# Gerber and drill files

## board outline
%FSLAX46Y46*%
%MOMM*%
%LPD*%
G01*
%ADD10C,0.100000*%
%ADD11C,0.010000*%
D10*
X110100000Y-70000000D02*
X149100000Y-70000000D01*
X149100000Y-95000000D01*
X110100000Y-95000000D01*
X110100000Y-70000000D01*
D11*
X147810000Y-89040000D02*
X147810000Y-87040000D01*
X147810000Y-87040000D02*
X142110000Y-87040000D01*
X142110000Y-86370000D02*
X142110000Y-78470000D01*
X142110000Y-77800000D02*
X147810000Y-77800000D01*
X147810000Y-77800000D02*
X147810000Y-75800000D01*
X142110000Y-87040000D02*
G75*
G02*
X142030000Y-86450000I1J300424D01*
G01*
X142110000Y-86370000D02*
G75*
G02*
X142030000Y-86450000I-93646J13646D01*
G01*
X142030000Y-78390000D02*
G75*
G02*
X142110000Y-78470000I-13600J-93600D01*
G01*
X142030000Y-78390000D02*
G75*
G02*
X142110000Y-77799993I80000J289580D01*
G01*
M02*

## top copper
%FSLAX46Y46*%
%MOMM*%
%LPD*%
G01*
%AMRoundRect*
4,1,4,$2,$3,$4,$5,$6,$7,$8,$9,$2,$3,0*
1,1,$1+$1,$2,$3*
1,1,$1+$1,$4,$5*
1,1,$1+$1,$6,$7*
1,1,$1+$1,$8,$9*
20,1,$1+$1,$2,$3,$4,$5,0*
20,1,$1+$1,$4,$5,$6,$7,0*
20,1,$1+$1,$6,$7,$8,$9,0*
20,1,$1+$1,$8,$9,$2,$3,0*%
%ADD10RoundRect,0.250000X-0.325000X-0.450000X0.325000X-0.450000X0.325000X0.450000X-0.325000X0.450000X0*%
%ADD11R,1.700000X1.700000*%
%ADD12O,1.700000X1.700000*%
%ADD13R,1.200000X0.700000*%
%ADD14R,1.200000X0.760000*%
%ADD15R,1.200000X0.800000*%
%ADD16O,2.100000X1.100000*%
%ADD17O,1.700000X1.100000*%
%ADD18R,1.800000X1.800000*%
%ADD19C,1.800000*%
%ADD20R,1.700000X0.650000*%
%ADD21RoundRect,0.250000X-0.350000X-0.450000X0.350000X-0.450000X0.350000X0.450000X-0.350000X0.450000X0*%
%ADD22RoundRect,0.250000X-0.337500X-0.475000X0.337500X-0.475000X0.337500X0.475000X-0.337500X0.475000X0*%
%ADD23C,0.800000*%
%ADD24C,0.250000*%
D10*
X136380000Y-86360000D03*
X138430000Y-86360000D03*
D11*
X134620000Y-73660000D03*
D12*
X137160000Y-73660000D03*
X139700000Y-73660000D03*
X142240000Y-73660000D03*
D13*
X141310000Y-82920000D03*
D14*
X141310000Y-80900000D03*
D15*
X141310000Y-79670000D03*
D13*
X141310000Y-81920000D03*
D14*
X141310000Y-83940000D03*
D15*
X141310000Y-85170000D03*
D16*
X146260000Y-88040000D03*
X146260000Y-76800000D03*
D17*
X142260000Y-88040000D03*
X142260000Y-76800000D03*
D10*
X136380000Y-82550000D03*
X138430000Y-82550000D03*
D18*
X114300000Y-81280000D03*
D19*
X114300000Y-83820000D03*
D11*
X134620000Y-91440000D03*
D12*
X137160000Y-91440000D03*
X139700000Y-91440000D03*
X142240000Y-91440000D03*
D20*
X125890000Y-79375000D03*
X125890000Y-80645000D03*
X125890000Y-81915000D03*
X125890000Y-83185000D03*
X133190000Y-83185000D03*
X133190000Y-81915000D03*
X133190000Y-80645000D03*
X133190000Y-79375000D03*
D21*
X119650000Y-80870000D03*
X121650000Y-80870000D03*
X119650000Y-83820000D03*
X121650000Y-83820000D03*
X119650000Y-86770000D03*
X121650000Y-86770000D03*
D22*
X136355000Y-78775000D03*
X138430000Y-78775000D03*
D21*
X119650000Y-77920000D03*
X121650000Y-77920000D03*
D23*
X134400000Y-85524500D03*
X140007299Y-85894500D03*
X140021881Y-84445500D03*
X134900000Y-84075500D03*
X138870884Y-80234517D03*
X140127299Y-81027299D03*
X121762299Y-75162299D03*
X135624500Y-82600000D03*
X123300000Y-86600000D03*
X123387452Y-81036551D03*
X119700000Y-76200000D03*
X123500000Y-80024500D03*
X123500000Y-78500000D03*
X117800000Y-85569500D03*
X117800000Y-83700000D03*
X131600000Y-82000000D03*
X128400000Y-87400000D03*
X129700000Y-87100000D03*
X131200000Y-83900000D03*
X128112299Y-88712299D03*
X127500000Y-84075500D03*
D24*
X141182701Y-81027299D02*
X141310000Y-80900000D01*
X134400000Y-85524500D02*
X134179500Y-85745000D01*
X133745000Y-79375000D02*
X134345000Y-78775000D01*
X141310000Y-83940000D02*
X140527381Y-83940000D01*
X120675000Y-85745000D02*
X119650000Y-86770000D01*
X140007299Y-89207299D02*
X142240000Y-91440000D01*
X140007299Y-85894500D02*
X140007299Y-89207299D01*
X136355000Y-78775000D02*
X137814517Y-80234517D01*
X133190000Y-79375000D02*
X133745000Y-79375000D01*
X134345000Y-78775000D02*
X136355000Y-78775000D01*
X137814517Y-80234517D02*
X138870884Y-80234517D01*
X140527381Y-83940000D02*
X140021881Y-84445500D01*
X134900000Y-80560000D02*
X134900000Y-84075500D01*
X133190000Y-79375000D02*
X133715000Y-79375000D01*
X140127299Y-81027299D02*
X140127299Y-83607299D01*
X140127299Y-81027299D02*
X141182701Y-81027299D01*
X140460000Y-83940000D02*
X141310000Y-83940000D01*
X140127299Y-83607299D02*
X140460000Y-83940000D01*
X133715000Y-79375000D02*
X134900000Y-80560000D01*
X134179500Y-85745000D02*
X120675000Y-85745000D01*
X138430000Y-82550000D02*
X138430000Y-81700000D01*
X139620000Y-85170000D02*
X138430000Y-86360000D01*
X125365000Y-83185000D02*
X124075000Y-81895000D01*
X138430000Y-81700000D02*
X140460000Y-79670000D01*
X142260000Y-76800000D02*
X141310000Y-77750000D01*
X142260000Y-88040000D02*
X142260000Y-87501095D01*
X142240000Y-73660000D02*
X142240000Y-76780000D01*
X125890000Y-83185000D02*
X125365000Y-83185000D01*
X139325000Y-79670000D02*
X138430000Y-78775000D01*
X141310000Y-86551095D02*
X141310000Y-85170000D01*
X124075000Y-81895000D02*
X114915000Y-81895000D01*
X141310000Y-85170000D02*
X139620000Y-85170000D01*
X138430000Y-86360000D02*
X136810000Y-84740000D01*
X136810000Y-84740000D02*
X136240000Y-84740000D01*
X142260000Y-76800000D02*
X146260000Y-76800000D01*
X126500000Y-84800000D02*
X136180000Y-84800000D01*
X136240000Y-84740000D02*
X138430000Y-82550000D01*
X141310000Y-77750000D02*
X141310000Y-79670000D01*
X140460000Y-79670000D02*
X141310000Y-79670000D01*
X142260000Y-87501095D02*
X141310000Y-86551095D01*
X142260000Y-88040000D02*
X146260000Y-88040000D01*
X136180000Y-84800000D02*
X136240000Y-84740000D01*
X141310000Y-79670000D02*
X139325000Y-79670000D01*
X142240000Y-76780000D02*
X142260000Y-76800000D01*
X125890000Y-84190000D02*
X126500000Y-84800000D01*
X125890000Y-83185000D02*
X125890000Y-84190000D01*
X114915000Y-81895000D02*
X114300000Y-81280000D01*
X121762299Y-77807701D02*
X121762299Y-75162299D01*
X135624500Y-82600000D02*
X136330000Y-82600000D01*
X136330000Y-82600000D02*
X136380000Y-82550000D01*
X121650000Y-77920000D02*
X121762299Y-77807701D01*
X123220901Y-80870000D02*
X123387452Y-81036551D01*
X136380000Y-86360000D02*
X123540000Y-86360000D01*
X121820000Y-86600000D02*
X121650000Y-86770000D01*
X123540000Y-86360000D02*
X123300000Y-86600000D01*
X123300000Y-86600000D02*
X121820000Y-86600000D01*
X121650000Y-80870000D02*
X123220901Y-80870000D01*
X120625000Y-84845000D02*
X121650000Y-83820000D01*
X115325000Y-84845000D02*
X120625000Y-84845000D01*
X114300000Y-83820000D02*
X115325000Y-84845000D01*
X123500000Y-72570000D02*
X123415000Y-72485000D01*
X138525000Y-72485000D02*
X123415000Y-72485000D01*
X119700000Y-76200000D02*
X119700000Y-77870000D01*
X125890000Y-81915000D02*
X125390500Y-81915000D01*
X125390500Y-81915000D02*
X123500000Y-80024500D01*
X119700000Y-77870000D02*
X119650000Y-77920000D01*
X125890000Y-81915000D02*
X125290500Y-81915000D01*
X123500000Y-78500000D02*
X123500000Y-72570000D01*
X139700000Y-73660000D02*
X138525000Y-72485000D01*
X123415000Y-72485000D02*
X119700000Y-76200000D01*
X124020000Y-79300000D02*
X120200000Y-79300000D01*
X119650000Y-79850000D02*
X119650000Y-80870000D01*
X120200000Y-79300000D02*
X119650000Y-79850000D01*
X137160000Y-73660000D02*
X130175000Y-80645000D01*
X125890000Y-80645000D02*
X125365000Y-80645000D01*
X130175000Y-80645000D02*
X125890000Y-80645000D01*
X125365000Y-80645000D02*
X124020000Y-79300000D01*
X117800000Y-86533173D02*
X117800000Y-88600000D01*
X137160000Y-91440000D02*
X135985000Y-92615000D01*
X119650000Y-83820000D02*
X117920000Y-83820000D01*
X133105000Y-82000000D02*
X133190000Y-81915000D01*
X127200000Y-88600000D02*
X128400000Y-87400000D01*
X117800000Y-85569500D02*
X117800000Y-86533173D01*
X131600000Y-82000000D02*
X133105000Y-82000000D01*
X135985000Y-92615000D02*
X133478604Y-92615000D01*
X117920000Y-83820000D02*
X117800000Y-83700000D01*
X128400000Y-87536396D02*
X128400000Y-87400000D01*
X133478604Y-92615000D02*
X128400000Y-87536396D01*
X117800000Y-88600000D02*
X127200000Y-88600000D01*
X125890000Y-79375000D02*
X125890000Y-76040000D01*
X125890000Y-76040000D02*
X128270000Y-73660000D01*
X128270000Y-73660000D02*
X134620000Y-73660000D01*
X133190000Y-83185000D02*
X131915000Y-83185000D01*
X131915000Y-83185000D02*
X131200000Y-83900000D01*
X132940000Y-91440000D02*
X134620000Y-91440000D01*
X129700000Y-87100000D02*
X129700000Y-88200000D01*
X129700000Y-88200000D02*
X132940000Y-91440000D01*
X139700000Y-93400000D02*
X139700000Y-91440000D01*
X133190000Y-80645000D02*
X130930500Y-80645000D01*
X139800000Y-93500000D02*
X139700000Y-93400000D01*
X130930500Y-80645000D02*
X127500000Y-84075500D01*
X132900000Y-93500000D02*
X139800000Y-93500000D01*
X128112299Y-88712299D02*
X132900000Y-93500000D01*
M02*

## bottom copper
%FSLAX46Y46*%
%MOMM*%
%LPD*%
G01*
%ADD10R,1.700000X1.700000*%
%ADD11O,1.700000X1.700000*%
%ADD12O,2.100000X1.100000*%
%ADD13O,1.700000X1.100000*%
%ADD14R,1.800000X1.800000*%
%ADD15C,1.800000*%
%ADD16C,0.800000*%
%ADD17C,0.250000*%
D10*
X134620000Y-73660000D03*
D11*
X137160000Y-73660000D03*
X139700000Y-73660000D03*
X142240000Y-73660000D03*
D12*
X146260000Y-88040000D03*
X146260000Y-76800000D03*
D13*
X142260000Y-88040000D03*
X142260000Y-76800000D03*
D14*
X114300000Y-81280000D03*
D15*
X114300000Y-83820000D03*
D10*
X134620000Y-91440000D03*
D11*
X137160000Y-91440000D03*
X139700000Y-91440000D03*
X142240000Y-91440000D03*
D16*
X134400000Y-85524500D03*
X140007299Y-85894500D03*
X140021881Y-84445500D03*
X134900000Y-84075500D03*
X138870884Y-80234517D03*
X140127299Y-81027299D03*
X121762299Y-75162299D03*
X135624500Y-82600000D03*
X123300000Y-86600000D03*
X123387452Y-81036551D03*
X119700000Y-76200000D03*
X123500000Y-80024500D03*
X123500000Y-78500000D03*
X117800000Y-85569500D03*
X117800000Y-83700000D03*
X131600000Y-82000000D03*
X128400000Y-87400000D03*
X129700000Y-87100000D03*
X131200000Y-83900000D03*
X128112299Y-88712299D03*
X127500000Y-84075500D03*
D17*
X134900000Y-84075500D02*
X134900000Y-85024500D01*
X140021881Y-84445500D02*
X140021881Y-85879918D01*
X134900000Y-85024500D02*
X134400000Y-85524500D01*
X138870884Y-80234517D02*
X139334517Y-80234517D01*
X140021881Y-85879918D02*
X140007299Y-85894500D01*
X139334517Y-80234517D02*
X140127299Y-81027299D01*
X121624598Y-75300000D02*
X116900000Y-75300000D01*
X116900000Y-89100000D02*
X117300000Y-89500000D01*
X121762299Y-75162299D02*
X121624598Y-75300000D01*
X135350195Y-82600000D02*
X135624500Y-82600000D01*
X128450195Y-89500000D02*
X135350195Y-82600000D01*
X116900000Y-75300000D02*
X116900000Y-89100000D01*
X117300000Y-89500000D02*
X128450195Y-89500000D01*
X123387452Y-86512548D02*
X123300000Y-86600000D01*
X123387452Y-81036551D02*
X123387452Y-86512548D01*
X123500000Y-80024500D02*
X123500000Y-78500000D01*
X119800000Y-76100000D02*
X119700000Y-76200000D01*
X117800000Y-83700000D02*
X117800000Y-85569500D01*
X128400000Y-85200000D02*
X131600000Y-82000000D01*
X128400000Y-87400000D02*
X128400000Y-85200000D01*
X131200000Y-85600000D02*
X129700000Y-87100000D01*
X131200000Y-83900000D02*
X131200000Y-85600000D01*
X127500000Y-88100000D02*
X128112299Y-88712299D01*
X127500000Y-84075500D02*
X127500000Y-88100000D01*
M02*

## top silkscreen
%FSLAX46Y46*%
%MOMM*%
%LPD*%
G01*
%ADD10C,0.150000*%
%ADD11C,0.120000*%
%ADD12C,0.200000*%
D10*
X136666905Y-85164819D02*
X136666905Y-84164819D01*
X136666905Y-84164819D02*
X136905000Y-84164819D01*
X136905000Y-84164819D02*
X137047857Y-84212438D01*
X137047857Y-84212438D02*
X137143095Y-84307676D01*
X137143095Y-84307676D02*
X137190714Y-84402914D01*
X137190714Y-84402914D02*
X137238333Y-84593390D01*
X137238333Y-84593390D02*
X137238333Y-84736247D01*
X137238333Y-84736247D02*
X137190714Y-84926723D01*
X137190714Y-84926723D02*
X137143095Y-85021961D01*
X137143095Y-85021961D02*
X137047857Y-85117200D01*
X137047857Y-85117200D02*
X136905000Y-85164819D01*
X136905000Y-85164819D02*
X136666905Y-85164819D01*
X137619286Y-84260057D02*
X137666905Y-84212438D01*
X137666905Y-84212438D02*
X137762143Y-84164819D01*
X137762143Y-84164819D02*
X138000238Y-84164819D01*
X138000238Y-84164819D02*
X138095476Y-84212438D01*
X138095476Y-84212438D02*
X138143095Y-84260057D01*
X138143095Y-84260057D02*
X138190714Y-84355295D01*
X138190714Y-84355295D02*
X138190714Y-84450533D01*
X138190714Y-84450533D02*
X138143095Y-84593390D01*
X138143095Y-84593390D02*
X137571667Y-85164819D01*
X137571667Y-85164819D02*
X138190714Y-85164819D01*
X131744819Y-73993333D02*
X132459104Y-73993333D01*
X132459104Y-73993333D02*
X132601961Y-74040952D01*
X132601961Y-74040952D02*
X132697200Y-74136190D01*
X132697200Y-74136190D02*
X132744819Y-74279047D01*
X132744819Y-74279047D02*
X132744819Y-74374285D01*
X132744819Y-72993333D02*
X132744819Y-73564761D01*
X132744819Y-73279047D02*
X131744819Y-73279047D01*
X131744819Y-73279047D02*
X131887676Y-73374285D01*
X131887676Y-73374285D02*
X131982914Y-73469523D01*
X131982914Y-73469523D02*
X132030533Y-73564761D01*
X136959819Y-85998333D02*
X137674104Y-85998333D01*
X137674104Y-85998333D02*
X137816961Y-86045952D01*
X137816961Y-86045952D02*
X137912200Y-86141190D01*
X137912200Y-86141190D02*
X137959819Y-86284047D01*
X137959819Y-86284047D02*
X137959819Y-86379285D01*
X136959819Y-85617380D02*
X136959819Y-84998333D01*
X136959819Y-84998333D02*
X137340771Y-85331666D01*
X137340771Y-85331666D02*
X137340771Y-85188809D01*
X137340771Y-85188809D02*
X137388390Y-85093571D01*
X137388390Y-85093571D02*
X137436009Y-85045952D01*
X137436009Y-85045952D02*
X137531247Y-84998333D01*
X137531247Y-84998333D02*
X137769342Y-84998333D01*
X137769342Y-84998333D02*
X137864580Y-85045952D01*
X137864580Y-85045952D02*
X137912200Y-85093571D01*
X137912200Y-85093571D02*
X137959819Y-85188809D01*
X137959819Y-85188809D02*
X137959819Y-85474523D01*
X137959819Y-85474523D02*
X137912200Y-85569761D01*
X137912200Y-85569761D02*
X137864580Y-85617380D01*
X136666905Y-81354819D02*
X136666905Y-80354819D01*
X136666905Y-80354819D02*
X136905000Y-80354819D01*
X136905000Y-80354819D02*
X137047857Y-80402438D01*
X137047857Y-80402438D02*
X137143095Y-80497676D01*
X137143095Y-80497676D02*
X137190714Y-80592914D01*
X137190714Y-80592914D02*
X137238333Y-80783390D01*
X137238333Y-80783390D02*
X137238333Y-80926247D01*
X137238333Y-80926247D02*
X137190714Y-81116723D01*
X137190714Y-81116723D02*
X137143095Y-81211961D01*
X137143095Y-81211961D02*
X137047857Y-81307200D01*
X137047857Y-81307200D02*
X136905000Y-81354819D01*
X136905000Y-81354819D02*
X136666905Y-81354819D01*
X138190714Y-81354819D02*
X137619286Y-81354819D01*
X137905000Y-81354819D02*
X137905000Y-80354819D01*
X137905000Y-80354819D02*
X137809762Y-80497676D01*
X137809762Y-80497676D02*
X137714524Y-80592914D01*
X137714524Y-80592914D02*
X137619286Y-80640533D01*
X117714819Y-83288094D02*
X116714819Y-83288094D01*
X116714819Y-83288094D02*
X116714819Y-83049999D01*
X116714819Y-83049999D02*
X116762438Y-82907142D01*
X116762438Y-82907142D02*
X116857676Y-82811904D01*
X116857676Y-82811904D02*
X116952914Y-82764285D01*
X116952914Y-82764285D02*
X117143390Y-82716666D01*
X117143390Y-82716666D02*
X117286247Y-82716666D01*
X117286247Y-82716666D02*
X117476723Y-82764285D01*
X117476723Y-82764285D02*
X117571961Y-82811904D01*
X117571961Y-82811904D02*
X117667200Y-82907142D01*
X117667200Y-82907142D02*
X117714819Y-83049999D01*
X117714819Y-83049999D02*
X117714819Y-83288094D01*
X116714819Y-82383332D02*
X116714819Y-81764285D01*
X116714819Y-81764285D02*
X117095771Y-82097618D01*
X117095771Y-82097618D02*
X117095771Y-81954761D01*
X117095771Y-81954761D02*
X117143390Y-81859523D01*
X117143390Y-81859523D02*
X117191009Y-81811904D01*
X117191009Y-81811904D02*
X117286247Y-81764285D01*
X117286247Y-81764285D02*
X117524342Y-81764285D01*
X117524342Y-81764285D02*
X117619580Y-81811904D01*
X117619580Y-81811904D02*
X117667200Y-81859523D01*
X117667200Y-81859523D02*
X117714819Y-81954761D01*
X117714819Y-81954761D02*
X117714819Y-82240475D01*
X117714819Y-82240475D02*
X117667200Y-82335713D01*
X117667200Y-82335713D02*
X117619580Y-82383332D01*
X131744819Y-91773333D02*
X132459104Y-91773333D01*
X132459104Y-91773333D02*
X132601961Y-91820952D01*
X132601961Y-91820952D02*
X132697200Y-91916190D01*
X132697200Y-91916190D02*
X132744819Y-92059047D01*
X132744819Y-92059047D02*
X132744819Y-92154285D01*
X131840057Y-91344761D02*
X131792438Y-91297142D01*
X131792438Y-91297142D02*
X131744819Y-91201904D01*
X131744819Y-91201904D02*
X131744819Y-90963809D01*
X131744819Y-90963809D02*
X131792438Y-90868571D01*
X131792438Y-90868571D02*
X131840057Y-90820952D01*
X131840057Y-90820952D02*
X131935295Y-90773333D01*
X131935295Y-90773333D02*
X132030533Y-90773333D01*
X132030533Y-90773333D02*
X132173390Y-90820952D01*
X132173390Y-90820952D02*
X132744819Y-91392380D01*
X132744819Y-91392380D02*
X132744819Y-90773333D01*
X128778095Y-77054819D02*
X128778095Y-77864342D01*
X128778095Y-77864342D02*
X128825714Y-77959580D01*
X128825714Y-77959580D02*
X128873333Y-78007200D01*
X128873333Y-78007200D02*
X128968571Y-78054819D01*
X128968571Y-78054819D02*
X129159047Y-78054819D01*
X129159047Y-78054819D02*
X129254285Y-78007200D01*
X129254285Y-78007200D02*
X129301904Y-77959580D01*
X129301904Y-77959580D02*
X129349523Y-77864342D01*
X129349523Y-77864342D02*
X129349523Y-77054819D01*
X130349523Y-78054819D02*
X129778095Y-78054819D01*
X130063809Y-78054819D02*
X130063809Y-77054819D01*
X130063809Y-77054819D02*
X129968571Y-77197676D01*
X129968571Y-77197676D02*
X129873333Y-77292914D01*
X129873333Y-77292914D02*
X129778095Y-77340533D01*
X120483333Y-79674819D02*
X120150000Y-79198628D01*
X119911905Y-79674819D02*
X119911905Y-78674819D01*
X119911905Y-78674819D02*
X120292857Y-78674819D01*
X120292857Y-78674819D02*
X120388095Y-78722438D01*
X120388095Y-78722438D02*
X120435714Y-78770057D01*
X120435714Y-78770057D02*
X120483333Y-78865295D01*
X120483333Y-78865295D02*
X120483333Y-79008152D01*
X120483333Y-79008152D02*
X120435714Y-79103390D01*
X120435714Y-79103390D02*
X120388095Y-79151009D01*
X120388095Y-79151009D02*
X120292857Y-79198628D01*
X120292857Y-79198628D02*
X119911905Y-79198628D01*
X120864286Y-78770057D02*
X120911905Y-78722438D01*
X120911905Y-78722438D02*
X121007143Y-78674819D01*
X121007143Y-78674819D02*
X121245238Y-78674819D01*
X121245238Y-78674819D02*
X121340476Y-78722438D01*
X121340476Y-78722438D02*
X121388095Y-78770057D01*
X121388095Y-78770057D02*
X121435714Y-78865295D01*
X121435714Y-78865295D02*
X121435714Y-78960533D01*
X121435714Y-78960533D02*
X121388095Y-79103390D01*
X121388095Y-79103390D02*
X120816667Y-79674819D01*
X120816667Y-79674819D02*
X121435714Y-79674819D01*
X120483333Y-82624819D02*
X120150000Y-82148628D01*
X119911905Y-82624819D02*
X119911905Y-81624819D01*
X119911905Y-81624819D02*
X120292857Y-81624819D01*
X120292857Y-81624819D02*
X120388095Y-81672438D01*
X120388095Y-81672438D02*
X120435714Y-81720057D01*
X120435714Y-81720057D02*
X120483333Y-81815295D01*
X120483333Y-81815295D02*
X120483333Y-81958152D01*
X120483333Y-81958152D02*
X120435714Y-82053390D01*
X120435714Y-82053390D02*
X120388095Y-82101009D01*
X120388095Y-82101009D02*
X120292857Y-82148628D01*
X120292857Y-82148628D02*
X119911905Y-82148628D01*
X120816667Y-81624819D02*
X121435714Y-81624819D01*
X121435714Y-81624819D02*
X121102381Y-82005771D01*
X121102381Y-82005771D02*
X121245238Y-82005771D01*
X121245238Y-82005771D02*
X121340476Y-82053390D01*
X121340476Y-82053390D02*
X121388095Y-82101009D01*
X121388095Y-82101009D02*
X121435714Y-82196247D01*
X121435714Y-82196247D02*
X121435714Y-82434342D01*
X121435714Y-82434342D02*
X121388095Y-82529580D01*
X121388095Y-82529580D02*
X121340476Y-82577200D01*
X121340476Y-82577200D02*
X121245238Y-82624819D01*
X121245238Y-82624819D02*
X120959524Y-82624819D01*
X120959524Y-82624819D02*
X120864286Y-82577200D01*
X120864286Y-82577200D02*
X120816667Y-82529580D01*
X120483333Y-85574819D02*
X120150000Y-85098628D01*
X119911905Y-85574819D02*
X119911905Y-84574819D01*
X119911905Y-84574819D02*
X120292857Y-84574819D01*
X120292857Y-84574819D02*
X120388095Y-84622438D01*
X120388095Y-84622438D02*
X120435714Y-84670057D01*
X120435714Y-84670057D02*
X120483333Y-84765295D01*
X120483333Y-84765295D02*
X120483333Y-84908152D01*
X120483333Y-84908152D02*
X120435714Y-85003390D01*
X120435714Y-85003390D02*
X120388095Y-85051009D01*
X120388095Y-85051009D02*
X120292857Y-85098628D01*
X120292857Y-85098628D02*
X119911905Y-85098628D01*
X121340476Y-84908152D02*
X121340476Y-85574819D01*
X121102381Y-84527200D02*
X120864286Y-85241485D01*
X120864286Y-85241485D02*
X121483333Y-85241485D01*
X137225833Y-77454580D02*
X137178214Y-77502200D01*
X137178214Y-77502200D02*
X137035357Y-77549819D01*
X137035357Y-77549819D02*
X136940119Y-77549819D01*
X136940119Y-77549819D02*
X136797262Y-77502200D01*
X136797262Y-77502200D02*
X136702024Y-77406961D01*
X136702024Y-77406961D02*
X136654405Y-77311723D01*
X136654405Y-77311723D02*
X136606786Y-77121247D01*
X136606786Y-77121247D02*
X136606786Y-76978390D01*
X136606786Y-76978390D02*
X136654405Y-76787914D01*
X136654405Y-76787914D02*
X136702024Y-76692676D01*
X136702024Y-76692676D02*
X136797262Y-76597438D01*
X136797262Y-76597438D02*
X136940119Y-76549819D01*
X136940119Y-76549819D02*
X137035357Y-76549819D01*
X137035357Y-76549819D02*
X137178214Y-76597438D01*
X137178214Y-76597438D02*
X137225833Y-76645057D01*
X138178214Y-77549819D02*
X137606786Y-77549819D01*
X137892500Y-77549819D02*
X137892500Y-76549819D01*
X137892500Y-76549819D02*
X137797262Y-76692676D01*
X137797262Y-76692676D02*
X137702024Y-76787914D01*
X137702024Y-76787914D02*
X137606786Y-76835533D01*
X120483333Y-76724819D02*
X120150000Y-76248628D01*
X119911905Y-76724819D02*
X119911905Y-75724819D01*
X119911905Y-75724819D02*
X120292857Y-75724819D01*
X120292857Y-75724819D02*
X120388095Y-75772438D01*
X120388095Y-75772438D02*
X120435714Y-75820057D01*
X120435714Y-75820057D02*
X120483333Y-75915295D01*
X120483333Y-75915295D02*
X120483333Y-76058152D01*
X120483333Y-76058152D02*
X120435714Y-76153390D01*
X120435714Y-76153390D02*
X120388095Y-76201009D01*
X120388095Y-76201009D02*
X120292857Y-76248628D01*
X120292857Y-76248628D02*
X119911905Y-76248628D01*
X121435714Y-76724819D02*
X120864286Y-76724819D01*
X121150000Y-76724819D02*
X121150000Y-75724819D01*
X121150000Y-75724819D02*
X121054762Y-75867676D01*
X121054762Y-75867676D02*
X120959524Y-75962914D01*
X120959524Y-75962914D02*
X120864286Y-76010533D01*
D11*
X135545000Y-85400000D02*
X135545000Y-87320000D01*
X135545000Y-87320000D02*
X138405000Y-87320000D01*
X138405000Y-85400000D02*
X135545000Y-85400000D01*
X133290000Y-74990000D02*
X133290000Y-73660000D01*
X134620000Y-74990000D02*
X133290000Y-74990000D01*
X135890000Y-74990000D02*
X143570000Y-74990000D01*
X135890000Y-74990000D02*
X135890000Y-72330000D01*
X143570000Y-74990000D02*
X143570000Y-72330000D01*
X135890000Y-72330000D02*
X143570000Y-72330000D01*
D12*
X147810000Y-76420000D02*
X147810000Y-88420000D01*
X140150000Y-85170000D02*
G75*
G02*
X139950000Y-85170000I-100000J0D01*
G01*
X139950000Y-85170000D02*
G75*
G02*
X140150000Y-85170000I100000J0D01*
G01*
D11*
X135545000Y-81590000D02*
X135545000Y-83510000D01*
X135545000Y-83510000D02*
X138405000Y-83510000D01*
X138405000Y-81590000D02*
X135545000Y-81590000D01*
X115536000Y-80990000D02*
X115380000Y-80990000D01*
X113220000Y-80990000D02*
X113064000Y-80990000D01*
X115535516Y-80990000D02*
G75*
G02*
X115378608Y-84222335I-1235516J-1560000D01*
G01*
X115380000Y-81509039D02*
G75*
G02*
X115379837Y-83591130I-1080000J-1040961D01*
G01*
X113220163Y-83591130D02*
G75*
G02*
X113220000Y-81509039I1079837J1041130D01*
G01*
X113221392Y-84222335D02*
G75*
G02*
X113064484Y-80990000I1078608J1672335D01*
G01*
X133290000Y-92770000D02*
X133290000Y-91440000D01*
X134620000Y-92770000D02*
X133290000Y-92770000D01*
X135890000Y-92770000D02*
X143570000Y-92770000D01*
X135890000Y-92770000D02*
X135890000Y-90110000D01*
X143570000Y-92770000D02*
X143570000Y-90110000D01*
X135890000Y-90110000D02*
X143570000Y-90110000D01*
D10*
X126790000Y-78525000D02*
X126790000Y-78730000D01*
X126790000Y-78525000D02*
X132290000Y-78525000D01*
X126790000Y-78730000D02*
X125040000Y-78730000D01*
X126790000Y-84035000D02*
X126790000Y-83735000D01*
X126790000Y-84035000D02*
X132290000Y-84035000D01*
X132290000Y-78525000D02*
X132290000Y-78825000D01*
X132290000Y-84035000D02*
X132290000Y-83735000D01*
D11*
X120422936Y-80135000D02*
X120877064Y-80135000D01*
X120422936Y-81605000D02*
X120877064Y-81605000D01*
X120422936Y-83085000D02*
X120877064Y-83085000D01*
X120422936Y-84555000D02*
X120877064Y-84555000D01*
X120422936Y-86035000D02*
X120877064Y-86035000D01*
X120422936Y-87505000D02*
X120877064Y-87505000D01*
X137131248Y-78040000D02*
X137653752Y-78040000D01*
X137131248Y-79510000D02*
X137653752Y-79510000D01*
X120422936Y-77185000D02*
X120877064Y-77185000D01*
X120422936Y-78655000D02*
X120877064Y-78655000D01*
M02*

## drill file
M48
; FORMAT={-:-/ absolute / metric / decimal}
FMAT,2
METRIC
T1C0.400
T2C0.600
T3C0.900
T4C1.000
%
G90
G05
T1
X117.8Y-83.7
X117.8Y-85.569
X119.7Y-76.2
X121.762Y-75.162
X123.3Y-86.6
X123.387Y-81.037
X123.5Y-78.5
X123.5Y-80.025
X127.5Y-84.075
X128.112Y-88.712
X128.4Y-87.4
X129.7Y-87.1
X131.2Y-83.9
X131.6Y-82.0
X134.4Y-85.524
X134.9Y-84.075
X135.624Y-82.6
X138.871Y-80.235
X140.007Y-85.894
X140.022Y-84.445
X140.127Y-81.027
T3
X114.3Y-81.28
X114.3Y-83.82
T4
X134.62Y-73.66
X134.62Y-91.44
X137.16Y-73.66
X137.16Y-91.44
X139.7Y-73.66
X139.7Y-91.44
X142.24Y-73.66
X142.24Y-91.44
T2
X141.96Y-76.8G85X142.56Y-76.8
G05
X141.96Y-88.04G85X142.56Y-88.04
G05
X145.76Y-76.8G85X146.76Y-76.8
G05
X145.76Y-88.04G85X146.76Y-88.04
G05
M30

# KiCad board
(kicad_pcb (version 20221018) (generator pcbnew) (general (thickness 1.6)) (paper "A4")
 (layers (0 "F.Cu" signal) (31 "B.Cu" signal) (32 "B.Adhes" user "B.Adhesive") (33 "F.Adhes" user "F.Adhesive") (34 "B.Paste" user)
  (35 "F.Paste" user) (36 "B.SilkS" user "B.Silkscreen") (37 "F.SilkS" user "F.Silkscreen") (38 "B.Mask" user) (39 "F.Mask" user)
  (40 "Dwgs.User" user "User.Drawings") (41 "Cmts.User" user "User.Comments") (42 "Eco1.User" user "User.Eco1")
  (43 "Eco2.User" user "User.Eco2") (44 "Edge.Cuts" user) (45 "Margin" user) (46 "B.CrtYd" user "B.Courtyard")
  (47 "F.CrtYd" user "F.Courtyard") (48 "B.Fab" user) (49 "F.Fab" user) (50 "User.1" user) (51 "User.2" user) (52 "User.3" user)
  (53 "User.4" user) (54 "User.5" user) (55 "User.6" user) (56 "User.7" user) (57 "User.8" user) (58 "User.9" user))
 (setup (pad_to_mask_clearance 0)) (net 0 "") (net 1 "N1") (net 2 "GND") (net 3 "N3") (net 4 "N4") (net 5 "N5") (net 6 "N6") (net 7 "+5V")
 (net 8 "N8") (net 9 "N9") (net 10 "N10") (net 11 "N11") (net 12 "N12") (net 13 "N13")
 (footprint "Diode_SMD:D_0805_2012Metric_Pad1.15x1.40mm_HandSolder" (layer "F.Cu") (at 137.405 86.36)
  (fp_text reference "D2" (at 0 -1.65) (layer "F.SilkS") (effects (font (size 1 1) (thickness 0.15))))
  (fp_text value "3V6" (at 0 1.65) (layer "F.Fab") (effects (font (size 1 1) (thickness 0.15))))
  (fp_line (start -1.86 -0.96) (end -1.86 0.96) (stroke (width 0.12) (type solid)) (layer "F.SilkS"))
  (fp_line (start -1.86 0.96) (end 1 0.96) (stroke (width 0.12) (type solid)) (layer "F.SilkS"))
  (fp_line (start 1 -0.96) (end -1.86 -0.96) (stroke (width 0.12) (type solid)) (layer "F.SilkS"))
  (pad "1" smd roundrect (at -1.025 0) (size 1.15 1.4) (layers "F.Cu" "F.Paste" "F.Mask") (roundrect_rratio 0.217391) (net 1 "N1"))
  (pad "2" smd roundrect (at 1.025 0) (size 1.15 1.4) (layers "F.Cu" "F.Paste" "F.Mask") (roundrect_rratio 0.217391) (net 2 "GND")))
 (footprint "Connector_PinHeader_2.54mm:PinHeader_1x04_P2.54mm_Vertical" (layer "F.Cu") (at 134.62 73.66 90)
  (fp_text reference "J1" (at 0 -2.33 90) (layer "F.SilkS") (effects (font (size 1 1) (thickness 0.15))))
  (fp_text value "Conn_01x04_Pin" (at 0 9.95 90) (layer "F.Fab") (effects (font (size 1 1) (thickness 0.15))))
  (fp_line (start -1.33 -1.33) (end 0 -1.33) (stroke (width 0.12) (type solid)) (layer "F.SilkS"))
  (fp_line (start -1.33 0) (end -1.33 -1.33) (stroke (width 0.12) (type solid)) (layer "F.SilkS"))
  (fp_line (start -1.33 1.27) (end -1.33 8.95) (stroke (width 0.12) (type solid)) (layer "F.SilkS"))
  (fp_line (start -1.33 1.27) (end 1.33 1.27) (stroke (width 0.12) (type solid)) (layer "F.SilkS"))
  (fp_line (start -1.33 8.95) (end 1.33 8.95) (stroke (width 0.12) (type solid)) (layer "F.SilkS"))
  (fp_line (start 1.33 1.27) (end 1.33 8.95) (stroke (width 0.12) (type solid)) (layer "F.SilkS"))
  (pad "1" thru_hole rect (at 0 0 90) (size 1.7 1.7) (drill 1) (layers "*.Cu" "*.Mask") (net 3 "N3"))
  (pad "2" thru_hole oval (at 0 2.54 90) (size 1.7 1.7) (drill 1) (layers "*.Cu" "*.Mask") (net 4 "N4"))
  (pad "3" thru_hole oval (at 0 5.08 90) (size 1.7 1.7) (drill 1) (layers "*.Cu" "*.Mask") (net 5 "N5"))
  (pad "4" thru_hole oval (at 0 7.62 90) (size 1.7 1.7) (drill 1) (layers "*.Cu" "*.Mask") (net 2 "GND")))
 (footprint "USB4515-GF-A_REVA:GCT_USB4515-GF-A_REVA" (layer "F.Cu") (at 146.26 82.42 90)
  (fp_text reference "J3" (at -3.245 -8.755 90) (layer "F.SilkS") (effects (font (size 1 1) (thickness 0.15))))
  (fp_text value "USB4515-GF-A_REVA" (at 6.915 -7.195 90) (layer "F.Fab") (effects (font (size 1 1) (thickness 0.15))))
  (fp_line (start 6 1.55) (end -6 1.55) (stroke (width 0.2) (type solid)) (layer "F.SilkS"))
  (fp_circle (center -2.75 -6.21) (end -2.65 -6.21) (stroke (width 0.2) (type solid)) (fill none) (layer "F.SilkS"))
  (fp_line (start -6.62 1.55) (end -4.62 1.55) (stroke (width 0.01) (type solid)) (layer "Edge.Cuts"))
  (fp_line (start -4.62 1.55) (end -4.62 -4.15) (stroke (width 0.01) (type solid)) (layer "Edge.Cuts"))
  (fp_line (start -3.95 -4.15) (end 3.95 -4.15) (stroke (width 0.01) (type solid)) (layer "Edge.Cuts"))
  (fp_line (start 4.62 -4.15) (end 4.62 1.55) (stroke (width 0.01) (type solid)) (layer "Edge.Cuts"))
  (fp_line (start 4.62 1.55) (end 6.62 1.55) (stroke (width 0.01) (type solid)) (layer "Edge.Cuts"))
  (fp_arc (start -4.62 -4.15) (mid -4.359942 -4.447699) (end -4.03 -4.23) (stroke (width 0.01) (type solid)) (layer "Edge.Cuts"))
  (fp_arc (start -3.95 -4.15) (mid -4.003271 -4.176729) (end -4.03 -4.23) (stroke (width 0.01) (type solid)) (layer "Edge.Cuts"))
  (fp_arc (start 4.03 -4.23) (mid 4.003271 -4.176729) (end 3.95 -4.15) (stroke (width 0.01) (type solid)) (layer "Edge.Cuts"))
  (fp_arc (start 4.03 -4.23) (mid 4.359942 -4.447699) (end 4.62 -4.15) (stroke (width 0.01) (type solid)) (layer "Edge.Cuts"))
  (pad "A5" smd rect (at -0.5 -4.95 90) (size 0.7 1.2) (layers "F.Cu" "F.Paste" "F.Mask") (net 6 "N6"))
  (pad "A9" smd rect (at 1.52 -4.95 90) (size 0.76 1.2) (layers "F.Cu" "F.Paste" "F.Mask") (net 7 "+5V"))
  (pad "A12" smd rect (at 2.75 -4.95 90) (size 0.8 1.2) (layers "F.Cu" "F.Paste" "F.Mask") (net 2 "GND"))
  (pad "B5" smd rect (at 0.5 -4.95 90) (size 0.7 1.2) (layers "F.Cu" "F.Paste" "F.Mask") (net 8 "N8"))
  (pad "B9" smd rect (at -1.52 -4.95 90) (size 0.76 1.2) (layers "F.Cu" "F.Paste" "F.Mask") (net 7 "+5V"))
  (pad "B12" smd rect (at -2.75 -4.95 90) (size 0.8 1.2) (layers "F.Cu" "F.Paste" "F.Mask") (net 2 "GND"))
  (pad "S1" thru_hole oval (at -5.62 0 90) (size 1.1 2.1) (drill oval 0.6 1.6) (layers "*.Cu" "*.Mask") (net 2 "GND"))
  (pad "S2" thru_hole oval (at 5.62 0 90) (size 1.1 2.1) (drill oval 0.6 1.6) (layers "*.Cu" "*.Mask") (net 2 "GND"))
  (pad "S3" thru_hole oval (at -5.62 -4 90) (size 1.1 1.7) (drill oval 0.6 1.2) (layers "*.Cu" "*.Mask") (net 2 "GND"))
  (pad "S4" thru_hole oval (at 5.62 -4 90) (size 1.1 1.7) (drill oval 0.6 1.2) (layers "*.Cu" "*.Mask") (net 2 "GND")))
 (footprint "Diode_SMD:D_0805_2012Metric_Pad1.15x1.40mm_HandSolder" (layer "F.Cu") (at 137.405 82.55)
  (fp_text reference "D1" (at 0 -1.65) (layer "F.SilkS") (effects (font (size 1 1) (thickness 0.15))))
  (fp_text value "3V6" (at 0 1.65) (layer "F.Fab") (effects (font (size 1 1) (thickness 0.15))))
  (fp_line (start -1.86 -0.96) (end -1.86 0.96) (stroke (width 0.12) (type solid)) (layer "F.SilkS"))
  (fp_line (start -1.86 0.96) (end 1 0.96) (stroke (width 0.12) (type solid)) (layer "F.SilkS"))
  (fp_line (start 1 -0.96) (end -1.86 -0.96) (stroke (width 0.12) (type solid)) (layer "F.SilkS"))
  (pad "1" smd roundrect (at -1.025 0) (size 1.15 1.4) (layers "F.Cu" "F.Paste" "F.Mask") (roundrect_rratio 0.217391) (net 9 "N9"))
  (pad "2" smd roundrect (at 1.025 0) (size 1.15 1.4) (layers "F.Cu" "F.Paste" "F.Mask") (roundrect_rratio 0.217391) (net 2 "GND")))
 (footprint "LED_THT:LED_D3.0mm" (layer "F.Cu") (at 114.3 81.28 -90)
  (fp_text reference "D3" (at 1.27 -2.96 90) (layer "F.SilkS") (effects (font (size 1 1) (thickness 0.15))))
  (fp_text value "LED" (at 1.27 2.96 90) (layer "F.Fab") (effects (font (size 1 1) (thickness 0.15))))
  (fp_line (start -0.29 -1.236) (end -0.29 -1.08) (stroke (width 0.12) (type solid)) (layer "F.SilkS"))
  (fp_line (start -0.29 1.08) (end -0.29 1.236) (stroke (width 0.12) (type solid)) (layer "F.SilkS"))
  (fp_arc (start -0.29 -1.235516) (mid 1.366487 -1.987659) (end 2.942335 -1.078608) (stroke (width 0.12) (type solid)) (layer "F.SilkS"))
  (fp_arc (start 0.229039 -1.08) (mid 1.270117 -1.5) (end 2.31113 -1.079837) (stroke (width 0.12) (type solid)) (layer "F.SilkS"))
  (fp_arc (start 2.31113 1.079837) (mid 1.270117 1.5) (end 0.229039 1.08) (stroke (width 0.12) (type solid)) (layer "F.SilkS"))
  (fp_arc (start 2.942335 1.078608) (mid 1.366487 1.987659) (end -0.29 1.235516) (stroke (width 0.12) (type solid)) (layer "F.SilkS"))
  (pad "1" thru_hole rect (at 0 0 270) (size 1.8 1.8) (drill 0.9) (layers "*.Cu" "*.Mask") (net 2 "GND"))
  (pad "2" thru_hole circle (at 2.54 0 270) (size 1.8 1.8) (drill 0.9) (layers "*.Cu" "*.Mask") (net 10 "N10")))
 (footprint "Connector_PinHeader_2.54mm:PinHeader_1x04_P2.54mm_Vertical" (layer "F.Cu") (at 134.62 91.44 90)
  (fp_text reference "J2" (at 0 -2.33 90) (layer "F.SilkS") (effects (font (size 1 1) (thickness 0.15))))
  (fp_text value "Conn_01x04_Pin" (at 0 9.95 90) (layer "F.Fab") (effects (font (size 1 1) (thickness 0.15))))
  (fp_line (start -1.33 -1.33) (end 0 -1.33) (stroke (width 0.12) (type solid)) (layer "F.SilkS"))
  (fp_line (start -1.33 0) (end -1.33 -1.33) (stroke (width 0.12) (type solid)) (layer "F.SilkS"))
  (fp_line (start -1.33 1.27) (end -1.33 8.95) (stroke (width 0.12) (type solid)) (layer "F.SilkS"))
  (fp_line (start -1.33 1.27) (end 1.33 1.27) (stroke (width 0.12) (type solid)) (layer "F.SilkS"))
  (fp_line (start -1.33 8.95) (end 1.33 8.95) (stroke (width 0.12) (type solid)) (layer "F.SilkS"))
  (fp_line (start 1.33 1.27) (end 1.33 8.95) (stroke (width 0.12) (type solid)) (layer "F.SilkS"))
  (pad "1" thru_hole rect (at 0 0 90) (size 1.7 1.7) (drill 1) (layers "*.Cu" "*.Mask") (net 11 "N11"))
  (pad "2" thru_hole oval (at 0 2.54 90) (size 1.7 1.7) (drill 1) (layers "*.Cu" "*.Mask") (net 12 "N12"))
  (pad "3" thru_hole oval (at 0 5.08 90) (size 1.7 1.7) (drill 1) (layers "*.Cu" "*.Mask") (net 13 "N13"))
  (pad "4" thru_hole oval (at 0 7.62 90) (size 1.7 1.7) (drill 1) (layers "*.Cu" "*.Mask") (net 7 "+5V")))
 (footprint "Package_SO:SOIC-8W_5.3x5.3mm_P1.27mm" (layer "F.Cu") (at 129.54 81.28)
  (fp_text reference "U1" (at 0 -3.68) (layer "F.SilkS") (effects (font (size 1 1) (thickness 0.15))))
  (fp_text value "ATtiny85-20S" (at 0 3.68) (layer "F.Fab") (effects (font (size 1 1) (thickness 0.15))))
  (fp_line (start -2.75 -2.755) (end -2.75 -2.55) (stroke (width 0.15) (type solid)) (layer "F.SilkS"))
  (fp_line (start -2.75 -2.755) (end 2.75 -2.755) (stroke (width 0.15) (type solid)) (layer "F.SilkS"))
  (fp_line (start -2.75 -2.55) (end -4.5 -2.55) (stroke (width 0.15) (type solid)) (layer "F.SilkS"))
  (fp_line (start -2.75 2.755) (end -2.75 2.455) (stroke (width 0.15) (type solid)) (layer "F.SilkS"))
  (fp_line (start -2.75 2.755) (end 2.75 2.755) (stroke (width 0.15) (type solid)) (layer "F.SilkS"))
  (fp_line (start 2.75 -2.755) (end 2.75 -2.455) (stroke (width 0.15) (type solid)) (layer "F.SilkS"))
  (fp_line (start 2.75 2.755) (end 2.75 2.455) (stroke (width 0.15) (type solid)) (layer "F.SilkS"))
  (pad "1" smd rect (at -3.65 -1.905) (size 1.7 0.65) (layers "F.Cu" "F.Paste" "F.Mask") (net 3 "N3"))
  (pad "2" smd rect (at -3.65 -0.635) (size 1.7 0.65) (layers "F.Cu" "F.Paste" "F.Mask") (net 4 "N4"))
  (pad "3" smd rect (at -3.65 0.635) (size 1.7 0.65) (layers "F.Cu" "F.Paste" "F.Mask") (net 5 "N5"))
  (pad "4" smd rect (at -3.65 1.905) (size 1.7 0.65) (layers "F.Cu" "F.Paste" "F.Mask") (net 2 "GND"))
  (pad "5" smd rect (at 3.65 1.905) (size 1.7 0.65) (layers "F.Cu" "F.Paste" "F.Mask") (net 11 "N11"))
  (pad "6" smd rect (at 3.65 0.635) (size 1.7 0.65) (layers "F.Cu" "F.Paste" "F.Mask") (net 12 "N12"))
  (pad "7" smd rect (at 3.65 -0.635) (size 1.7 0.65) (layers "F.Cu" "F.Paste" "F.Mask") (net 13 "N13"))
  (pad "8" smd rect (at 3.65 -1.905) (size 1.7 0.65) (layers "F.Cu" "F.Paste" "F.Mask") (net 7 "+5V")))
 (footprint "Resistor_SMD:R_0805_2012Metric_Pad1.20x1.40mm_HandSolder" (layer "F.Cu") (at 120.65 80.87)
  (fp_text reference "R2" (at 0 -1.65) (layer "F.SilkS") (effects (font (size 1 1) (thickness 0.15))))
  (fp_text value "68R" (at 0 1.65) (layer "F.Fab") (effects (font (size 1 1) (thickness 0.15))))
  (fp_line (start -0.227064 -0.735) (end 0.227064 -0.735) (stroke (width 0.12) (type solid)) (layer "F.SilkS"))
  (fp_line (start -0.227064 0.735) (end 0.227064 0.735) (stroke (width 0.12) (type solid)) (layer "F.SilkS"))
  (pad "1" smd roundrect (at -1 0) (size 1.2 1.4) (layers "F.Cu" "F.Paste" "F.Mask") (roundrect_rratio 0.208333) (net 4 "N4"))
  (pad "2" smd roundrect (at 1 0) (size 1.2 1.4) (layers "F.Cu" "F.Paste" "F.Mask") (roundrect_rratio 0.208333) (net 1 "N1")))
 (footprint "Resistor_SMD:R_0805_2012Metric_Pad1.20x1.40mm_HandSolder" (layer "F.Cu") (at 120.65 83.82)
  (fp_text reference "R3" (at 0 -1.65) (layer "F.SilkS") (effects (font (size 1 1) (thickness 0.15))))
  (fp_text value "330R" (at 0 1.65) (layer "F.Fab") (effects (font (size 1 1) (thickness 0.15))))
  (fp_line (start -0.227064 -0.735) (end 0.227064 -0.735) (stroke (width 0.12) (type solid)) (layer "F.SilkS"))
  (fp_line (start -0.227064 0.735) (end 0.227064 0.735) (stroke (width 0.12) (type solid)) (layer "F.SilkS"))
  (pad "1" smd roundrect (at -1 0) (size 1.2 1.4) (layers "F.Cu" "F.Paste" "F.Mask") (roundrect_rratio 0.208333) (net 12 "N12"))
  (pad "2" smd roundrect (at 1 0) (size 1.2 1.4) (layers "F.Cu" "F.Paste" "F.Mask") (roundrect_rratio 0.208333) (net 10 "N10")))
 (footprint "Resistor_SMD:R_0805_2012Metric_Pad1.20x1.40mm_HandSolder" (layer "F.Cu") (at 120.65 86.77)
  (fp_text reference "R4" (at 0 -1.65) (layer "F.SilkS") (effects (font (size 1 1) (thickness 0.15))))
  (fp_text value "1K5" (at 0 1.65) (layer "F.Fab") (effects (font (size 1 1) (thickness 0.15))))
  (fp_line (start -0.227064 -0.735) (end 0.227064 -0.735) (stroke (width 0.12) (type solid)) (layer "F.SilkS"))
  (fp_line (start -0.227064 0.735) (end 0.227064 0.735) (stroke (width 0.12) (type solid)) (layer "F.SilkS"))
  (pad "1" smd roundrect (at -1 0) (size 1.2 1.4) (layers "F.Cu" "F.Paste" "F.Mask") (roundrect_rratio 0.208333) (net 7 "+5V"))
  (pad "2" smd roundrect (at 1 0) (size 1.2 1.4) (layers "F.Cu" "F.Paste" "F.Mask") (roundrect_rratio 0.208333) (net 1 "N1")))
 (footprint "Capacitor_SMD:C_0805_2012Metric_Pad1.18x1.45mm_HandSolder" (layer "F.Cu") (at 137.3925 78.775)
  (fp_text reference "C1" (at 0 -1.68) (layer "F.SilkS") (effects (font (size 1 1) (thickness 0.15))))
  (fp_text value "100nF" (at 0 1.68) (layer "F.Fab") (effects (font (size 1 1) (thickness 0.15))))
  (fp_line (start -0.261252 -0.735) (end 0.261252 -0.735) (stroke (width 0.12) (type solid)) (layer "F.SilkS"))
  (fp_line (start -0.261252 0.735) (end 0.261252 0.735) (stroke (width 0.12) (type solid)) (layer "F.SilkS"))
  (pad "1" smd roundrect (at -1.0375 0) (size 1.175 1.45) (layers "F.Cu" "F.Paste" "F.Mask") (roundrect_rratio 0.212766) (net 7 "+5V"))
  (pad "2" smd roundrect (at 1.0375 0) (size 1.175 1.45) (layers "F.Cu" "F.Paste" "F.Mask") (roundrect_rratio 0.212766) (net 2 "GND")))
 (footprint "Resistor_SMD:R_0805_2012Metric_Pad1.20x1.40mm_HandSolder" (layer "F.Cu") (at 120.65 77.92)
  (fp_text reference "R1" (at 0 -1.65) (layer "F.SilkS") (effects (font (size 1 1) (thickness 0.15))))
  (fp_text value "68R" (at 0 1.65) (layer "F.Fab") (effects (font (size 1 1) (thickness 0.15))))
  (fp_line (start -0.227064 -0.735) (end 0.227064 -0.735) (stroke (width 0.12) (type solid)) (layer "F.SilkS"))
  (fp_line (start -0.227064 0.735) (end 0.227064 0.735) (stroke (width 0.12) (type solid)) (layer "F.SilkS"))
  (pad "1" smd roundrect (at -1 0) (size 1.2 1.4) (layers "F.Cu" "F.Paste" "F.Mask") (roundrect_rratio 0.208333) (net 5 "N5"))
  (pad "2" smd roundrect (at 1 0) (size 1.2 1.4) (layers "F.Cu" "F.Paste" "F.Mask") (roundrect_rratio 0.208333) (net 9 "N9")))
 (gr_rect (start 110.1 70) (end 149.1 95) (stroke (width 0.1) (type default)) (fill none) (layer "Edge.Cuts"))
 (segment (start 141.182701 81.027299) (end 141.31 80.9) (width 0.25) (layer "F.Cu") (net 7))
 (segment (start 134.4 85.5245) (end 134.1795 85.745) (width 0.25) (layer "F.Cu") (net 7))
 (segment (start 133.745 79.375) (end 134.345 78.775) (width 0.25) (layer "F.Cu") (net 7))
 (segment (start 141.31 83.94) (end 140.527381 83.94) (width 0.25) (layer "F.Cu") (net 7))
 (segment (start 120.675 85.745) (end 119.65 86.77) (width 0.25) (layer "F.Cu") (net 7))
 (segment (start 140.007299 89.207299) (end 142.24 91.44) (width 0.25) (layer "F.Cu") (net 7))
 (segment (start 140.007299 85.8945) (end 140.007299 89.207299) (width 0.25) (layer "F.Cu") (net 7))
 (segment (start 136.355 78.775) (end 137.814517 80.234517) (width 0.25) (layer "F.Cu") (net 7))
 (segment (start 133.19 79.375) (end 133.745 79.375) (width 0.25) (layer "F.Cu") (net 7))
 (segment (start 134.345 78.775) (end 136.355 78.775) (width 0.25) (layer "F.Cu") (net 7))
 (segment (start 137.814517 80.234517) (end 138.870884 80.234517) (width 0.25) (layer "F.Cu") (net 7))
 (segment (start 140.527381 83.94) (end 140.021881 84.4455) (width 0.25) (layer "F.Cu") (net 7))
 (segment (start 134.9 80.56) (end 134.9 84.0755) (width 0.25) (layer "F.Cu") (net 7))
 (segment (start 133.19 79.375) (end 133.715 79.375) (width 0.25) (layer "F.Cu") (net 7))
 (segment (start 140.127299 81.027299) (end 140.127299 83.607299) (width 0.25) (layer "F.Cu") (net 7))
 (segment (start 140.127299 81.027299) (end 141.182701 81.027299) (width 0.25) (layer "F.Cu") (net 7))
 (segment (start 140.46 83.94) (end 141.31 83.94) (width 0.25) (layer "F.Cu") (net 7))
 (segment (start 140.127299 83.607299) (end 140.46 83.94) (width 0.25) (layer "F.Cu") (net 7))
 (segment (start 133.715 79.375) (end 134.9 80.56) (width 0.25) (layer "F.Cu") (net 7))
 (segment (start 134.1795 85.745) (end 120.675 85.745) (width 0.25) (layer "F.Cu") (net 7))
 (via (at 134.4 85.5245) (size 0.8) (drill 0.4) (layers "F.Cu" "B.Cu") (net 7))
 (via (at 140.007299 85.8945) (size 0.8) (drill 0.4) (layers "F.Cu" "B.Cu") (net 7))
 (via (at 140.021881 84.4455) (size 0.8) (drill 0.4) (layers "F.Cu" "B.Cu") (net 7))
 (via (at 134.9 84.0755) (size 0.8) (drill 0.4) (layers "F.Cu" "B.Cu") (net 7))
 (via (at 138.870884 80.234517) (size 0.8) (drill 0.4) (layers "F.Cu" "B.Cu") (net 7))
 (via (at 140.127299 81.027299) (size 0.8) (drill 0.4) (layers "F.Cu" "B.Cu") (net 7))
 (segment (start 134.9 84.0755) (end 134.9 85.0245) (width 0.25) (layer "B.Cu") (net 7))
 (segment (start 140.021881 84.4455) (end 140.021881 85.879918) (width 0.25) (layer "B.Cu") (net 7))
 (segment (start 134.9 85.0245) (end 134.4 85.5245) (width 0.25) (layer "B.Cu") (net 7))
 (segment (start 138.870884 80.234517) (end 139.334517 80.234517) (width 0.25) (layer "B.Cu") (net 7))
 (segment (start 140.021881 85.879918) (end 140.007299 85.8945) (width 0.25) (layer "B.Cu") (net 7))
 (segment (start 139.334517 80.234517) (end 140.127299 81.027299) (width 0.25) (layer "B.Cu") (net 7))
 (segment (start 138.43 82.55) (end 138.43 81.7) (width 0.25) (layer "F.Cu") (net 2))
 (segment (start 139.62 85.17) (end 138.43 86.36) (width 0.25) (layer "F.Cu") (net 2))
 (segment (start 125.365 83.185) (end 124.075 81.895) (width 0.25) (layer "F.Cu") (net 2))
 (segment (start 138.43 81.7) (end 140.46 79.67) (width 0.25) (layer "F.Cu") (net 2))
 (segment (start 142.26 76.8) (end 141.31 77.75) (width 0.25) (layer "F.Cu") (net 2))
 (segment (start 142.26 88.04) (end 142.26 87.501095) (width 0.25) (layer "F.Cu") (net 2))
 (segment (start 142.24 73.66) (end 142.24 76.78) (width 0.25) (layer "F.Cu") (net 2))
 (segment (start 125.89 83.185) (end 125.365 83.185) (width 0.25) (layer "F.Cu") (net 2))
 (segment (start 139.325 79.67) (end 138.43 78.775) (width 0.25) (layer "F.Cu") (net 2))
 (segment (start 141.31 86.551095) (end 141.31 85.17) (width 0.25) (layer "F.Cu") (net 2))
 (segment (start 124.075 81.895) (end 114.915 81.895) (width 0.25) (layer "F.Cu") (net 2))
 (segment (start 141.31 85.17) (end 139.62 85.17) (width 0.25) (layer "F.Cu") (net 2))
 (segment (start 138.43 86.36) (end 136.81 84.74) (width 0.25) (layer "F.Cu") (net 2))
 (segment (start 136.81 84.74) (end 136.24 84.74) (width 0.25) (layer "F.Cu") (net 2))
 (segment (start 142.26 76.8) (end 146.26 76.8) (width 0.25) (layer "F.Cu") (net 2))
 (segment (start 126.5 84.8) (end 136.18 84.8) (width 0.25) (layer "F.Cu") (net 2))
 (segment (start 136.24 84.74) (end 138.43 82.55) (width 0.25) (layer "F.Cu") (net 2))
 (segment (start 141.31 77.75) (end 141.31 79.67) (width 0.25) (layer "F.Cu") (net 2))
 (segment (start 140.46 79.67) (end 141.31 79.67) (width 0.25) (layer "F.Cu") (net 2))
 (segment (start 142.26 87.501095) (end 141.31 86.551095) (width 0.25) (layer "F.Cu") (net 2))
 (segment (start 142.26 88.04) (end 146.26 88.04) (width 0.25) (layer "F.Cu") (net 2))
 (segment (start 136.18 84.8) (end 136.24 84.74) (width 0.25) (layer "F.Cu") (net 2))
 (segment (start 141.31 79.67) (end 139.325 79.67) (width 0.25) (layer "F.Cu") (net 2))
 (segment (start 142.24 76.78) (end 142.26 76.8) (width 0.25) (layer "F.Cu") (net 2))
 (segment (start 125.89 84.19) (end 126.5 84.8) (width 0.25) (layer "F.Cu") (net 2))
 (segment (start 125.89 83.185) (end 125.89 84.19) (width 0.25) (layer "F.Cu") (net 2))
 (segment (start 114.915 81.895) (end 114.3 81.28) (width 0.25) (layer "F.Cu") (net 2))
 (segment (start 121.762299 77.807701) (end 121.762299 75.162299) (width 0.25) (layer "F.Cu") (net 9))
 (segment (start 135.6245 82.6) (end 136.33 82.6) (width 0.25) (layer "F.Cu") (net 9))
 (segment (start 136.33 82.6) (end 136.38 82.55) (width 0.25) (layer "F.Cu") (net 9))
 (segment (start 121.65 77.92) (end 121.762299 77.807701) (width 0.25) (layer "F.Cu") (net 9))
 (via (at 121.762299 75.162299) (size 0.8) (drill 0.4) (layers "F.Cu" "B.Cu") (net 9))
 (via (at 135.6245 82.6) (size 0.8) (drill 0.4) (layers "F.Cu" "B.Cu") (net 9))
 (segment (start 121.624598 75.3) (end 116.9 75.3) (width 0.25) (layer "B.Cu") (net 9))
 (segment (start 116.9 89.1) (end 117.3 89.5) (width 0.25) (layer "B.Cu") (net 9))
 (segment (start 121.762299 75.162299) (end 121.624598 75.3) (width 0.25) (layer "B.Cu") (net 9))
 (segment (start 135.350195 82.6) (end 135.6245 82.6) (width 0.25) (layer "B.Cu") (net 9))
 (segment (start 128.450195 89.5) (end 135.350195 82.6) (width 0.25) (layer "B.Cu") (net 9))
 (segment (start 116.9 75.3) (end 116.9 89.1) (width 0.25) (layer "B.Cu") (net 9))
 (segment (start 117.3 89.5) (end 128.450195 89.5) (width 0.25) (layer "B.Cu") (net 9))
 (segment (start 123.220901 80.87) (end 123.387452 81.036551) (width 0.25) (layer "F.Cu") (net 1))
 (segment (start 136.38 86.36) (end 123.54 86.36) (width 0.25) (layer "F.Cu") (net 1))
 (segment (start 121.82 86.6) (end 121.65 86.77) (width 0.25) (layer "F.Cu") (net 1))
 (segment (start 123.54 86.36) (end 123.3 86.6) (width 0.25) (layer "F.Cu") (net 1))
 (segment (start 123.3 86.6) (end 121.82 86.6) (width 0.25) (layer "F.Cu") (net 1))
 (segment (start 121.65 80.87) (end 123.220901 80.87) (width 0.25) (layer "F.Cu") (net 1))
 (via (at 123.3 86.6) (size 0.8) (drill 0.4) (layers "F.Cu" "B.Cu") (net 1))
 (via (at 123.387452 81.036551) (size 0.8) (drill 0.4) (layers "F.Cu" "B.Cu") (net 1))
 (segment (start 123.387452 86.512548) (end 123.3 86.6) (width 0.25) (layer "B.Cu") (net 1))
 (segment (start 123.387452 81.036551) (end 123.387452 86.512548) (width 0.25) (layer "B.Cu") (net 1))
 (segment (start 120.625 84.845) (end 121.65 83.82) (width 0.25) (layer "F.Cu") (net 10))
 (segment (start 115.325 84.845) (end 120.625 84.845) (width 0.25) (layer "F.Cu") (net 10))
 (segment (start 114.3 83.82) (end 115.325 84.845) (width 0.25) (layer "F.Cu") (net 10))
 (segment (start 123.5 72.57) (end 123.415 72.485) (width 0.25) (layer "F.Cu") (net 5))
 (segment (start 138.525 72.485) (end 123.415 72.485) (width 0.25) (layer "F.Cu") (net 5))
 (segment (start 119.7 76.2) (end 119.7 77.87) (width 0.25) (layer "F.Cu") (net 5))
 (segment (start 125.89 81.915) (end 125.3905 81.915) (width 0.25) (layer "F.Cu") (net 5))
 (segment (start 125.3905 81.915) (end 123.5 80.0245) (width 0.25) (layer "F.Cu") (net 5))
 (segment (start 119.7 77.87) (end 119.65 77.92) (width 0.25) (layer "F.Cu") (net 5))
 (segment (start 125.89 81.915) (end 125.2905 81.915) (width 0.25) (layer "F.Cu") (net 5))
 (segment (start 123.5 78.5) (end 123.5 72.57) (width 0.25) (layer "F.Cu") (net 5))
 (segment (start 139.7 73.66) (end 138.525 72.485) (width 0.25) (layer "F.Cu") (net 5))
 (segment (start 123.415 72.485) (end 119.7 76.2) (width 0.25) (layer "F.Cu") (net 5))
 (via (at 119.7 76.2) (size 0.8) (drill 0.4) (layers "F.Cu" "B.Cu") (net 5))
 (via (at 123.5 80.0245) (size 0.8) (drill 0.4) (layers "F.Cu" "B.Cu") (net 5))
 (via (at 123.5 78.5) (size 0.8) (drill 0.4) (layers "F.Cu" "B.Cu") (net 5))
 (segment (start 123.5 80.0245) (end 123.5 78.5) (width 0.25) (layer "B.Cu") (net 5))
 (segment (start 119.8 76.1) (end 119.7 76.2) (width 0.25) (layer "B.Cu") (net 5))
 (segment (start 124.02 79.3) (end 120.2 79.3) (width 0.25) (layer "F.Cu") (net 4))
 (segment (start 119.65 79.85) (end 119.65 80.87) (width 0.25) (layer "F.Cu") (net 4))
 (segment (start 120.2 79.3) (end 119.65 79.85) (width 0.25) (layer "F.Cu") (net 4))
 (segment (start 137.16 73.66) (end 130.175 80.645) (width 0.25) (layer "F.Cu") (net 4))
 (segment (start 125.89 80.645) (end 125.365 80.645) (width 0.25) (layer "F.Cu") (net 4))
 (segment (start 130.175 80.645) (end 125.89 80.645) (width 0.25) (layer "F.Cu") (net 4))
 (segment (start 125.365 80.645) (end 124.02 79.3) (width 0.25) (layer "F.Cu") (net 4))
 (segment (start 117.8 86.533173) (end 117.8 88.6) (width 0.25) (layer "F.Cu") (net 12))
 (segment (start 137.16 91.44) (end 135.985 92.615) (width 0.25) (layer "F.Cu") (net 12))
 (segment (start 119.65 83.82) (end 117.92 83.82) (width 0.25) (layer "F.Cu") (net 12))
 (segment (start 133.105 82) (end 133.19 81.915) (width 0.25) (layer "F.Cu") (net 12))
 (segment (start 127.2 88.6) (end 128.4 87.4) (width 0.25) (layer "F.Cu") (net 12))
 (segment (start 117.8 85.5695) (end 117.8 86.533173) (width 0.25) (layer "F.Cu") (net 12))
 (segment (start 131.6 82) (end 133.105 82) (width 0.25) (layer "F.Cu") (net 12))
 (segment (start 135.985 92.615) (end 133.478604 92.615) (width 0.25) (layer "F.Cu") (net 12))
 (segment (start 117.92 83.82) (end 117.8 83.7) (width 0.25) (layer "F.Cu") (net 12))
 (segment (start 128.4 87.536396) (end 128.4 87.4) (width 0.25) (layer "F.Cu") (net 12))
 (segment (start 133.478604 92.615) (end 128.4 87.536396) (width 0.25) (layer "F.Cu") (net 12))
 (segment (start 117.8 88.6) (end 127.2 88.6) (width 0.25) (layer "F.Cu") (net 12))
 (via (at 117.8 85.5695) (size 0.8) (drill 0.4) (layers "F.Cu" "B.Cu") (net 12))
 (via (at 117.8 83.7) (size 0.8) (drill 0.4) (layers "F.Cu" "B.Cu") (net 12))
 (via (at 131.6 82) (size 0.8) (drill 0.4) (layers "F.Cu" "B.Cu") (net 12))
 (via (at 128.4 87.4) (size 0.8) (drill 0.4) (layers "F.Cu" "B.Cu") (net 12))
 (segment (start 117.8 83.7) (end 117.8 85.5695) (width 0.25) (layer "B.Cu") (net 12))
 (segment (start 128.4 85.2) (end 131.6 82) (width 0.25) (layer "B.Cu") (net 12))
 (segment (start 128.4 87.4) (end 128.4 85.2) (width 0.25) (layer "B.Cu") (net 12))
 (segment (start 125.89 79.375) (end 125.89 76.04) (width 0.25) (layer "F.Cu") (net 3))
 (segment (start 125.89 76.04) (end 128.27 73.66) (width 0.25) (layer "F.Cu") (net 3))
 (segment (start 128.27 73.66) (end 134.62 73.66) (width 0.25) (layer "F.Cu") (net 3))
 (segment (start 133.19 83.185) (end 131.915 83.185) (width 0.25) (layer "F.Cu") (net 11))
 (segment (start 131.915 83.185) (end 131.2 83.9) (width 0.25) (layer "F.Cu") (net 11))
 (segment (start 132.94 91.44) (end 134.62 91.44) (width 0.25) (layer "F.Cu") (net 11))
 (segment (start 129.7 87.1) (end 129.7 88.2) (width 0.25) (layer "F.Cu") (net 11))
 (segment (start 129.7 88.2) (end 132.94 91.44) (width 0.25) (layer "F.Cu") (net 11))
 (via (at 129.7 87.1) (size 0.8) (drill 0.4) (layers "F.Cu" "B.Cu") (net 11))
 (via (at 131.2 83.9) (size 0.8) (drill 0.4) (layers "F.Cu" "B.Cu") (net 11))
 (segment (start 131.2 85.6) (end 129.7 87.1) (width 0.25) (layer "B.Cu") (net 11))
 (segment (start 131.2 83.9) (end 131.2 85.6) (width 0.25) (layer "B.Cu") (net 11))
 (segment (start 139.7 93.4) (end 139.7 91.44) (width 0.25) (layer "F.Cu") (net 13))
 (segment (start 133.19 80.645) (end 130.9305 80.645) (width 0.25) (layer "F.Cu") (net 13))
 (segment (start 139.8 93.5) (end 139.7 93.4) (width 0.25) (layer "F.Cu") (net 13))
 (segment (start 130.9305 80.645) (end 127.5 84.0755) (width 0.25) (layer "F.Cu") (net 13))
 (segment (start 132.9 93.5) (end 139.8 93.5) (width 0.25) (layer "F.Cu") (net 13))
 (segment (start 128.112299 88.712299) (end 132.9 93.5) (width 0.25) (layer "F.Cu") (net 13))
 (via (at 128.112299 88.712299) (size 0.8) (drill 0.4) (layers "F.Cu" "B.Cu") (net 13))
 (via (at 127.5 84.0755) (size 0.8) (drill 0.4) (layers "F.Cu" "B.Cu") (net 13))
 (segment (start 127.5 88.1) (end 128.112299 88.712299) (width 0.25) (layer "B.Cu") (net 13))
 (segment (start 127.5 84.0755) (end 127.5 88.1) (width 0.25) (layer "B.Cu") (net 13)))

